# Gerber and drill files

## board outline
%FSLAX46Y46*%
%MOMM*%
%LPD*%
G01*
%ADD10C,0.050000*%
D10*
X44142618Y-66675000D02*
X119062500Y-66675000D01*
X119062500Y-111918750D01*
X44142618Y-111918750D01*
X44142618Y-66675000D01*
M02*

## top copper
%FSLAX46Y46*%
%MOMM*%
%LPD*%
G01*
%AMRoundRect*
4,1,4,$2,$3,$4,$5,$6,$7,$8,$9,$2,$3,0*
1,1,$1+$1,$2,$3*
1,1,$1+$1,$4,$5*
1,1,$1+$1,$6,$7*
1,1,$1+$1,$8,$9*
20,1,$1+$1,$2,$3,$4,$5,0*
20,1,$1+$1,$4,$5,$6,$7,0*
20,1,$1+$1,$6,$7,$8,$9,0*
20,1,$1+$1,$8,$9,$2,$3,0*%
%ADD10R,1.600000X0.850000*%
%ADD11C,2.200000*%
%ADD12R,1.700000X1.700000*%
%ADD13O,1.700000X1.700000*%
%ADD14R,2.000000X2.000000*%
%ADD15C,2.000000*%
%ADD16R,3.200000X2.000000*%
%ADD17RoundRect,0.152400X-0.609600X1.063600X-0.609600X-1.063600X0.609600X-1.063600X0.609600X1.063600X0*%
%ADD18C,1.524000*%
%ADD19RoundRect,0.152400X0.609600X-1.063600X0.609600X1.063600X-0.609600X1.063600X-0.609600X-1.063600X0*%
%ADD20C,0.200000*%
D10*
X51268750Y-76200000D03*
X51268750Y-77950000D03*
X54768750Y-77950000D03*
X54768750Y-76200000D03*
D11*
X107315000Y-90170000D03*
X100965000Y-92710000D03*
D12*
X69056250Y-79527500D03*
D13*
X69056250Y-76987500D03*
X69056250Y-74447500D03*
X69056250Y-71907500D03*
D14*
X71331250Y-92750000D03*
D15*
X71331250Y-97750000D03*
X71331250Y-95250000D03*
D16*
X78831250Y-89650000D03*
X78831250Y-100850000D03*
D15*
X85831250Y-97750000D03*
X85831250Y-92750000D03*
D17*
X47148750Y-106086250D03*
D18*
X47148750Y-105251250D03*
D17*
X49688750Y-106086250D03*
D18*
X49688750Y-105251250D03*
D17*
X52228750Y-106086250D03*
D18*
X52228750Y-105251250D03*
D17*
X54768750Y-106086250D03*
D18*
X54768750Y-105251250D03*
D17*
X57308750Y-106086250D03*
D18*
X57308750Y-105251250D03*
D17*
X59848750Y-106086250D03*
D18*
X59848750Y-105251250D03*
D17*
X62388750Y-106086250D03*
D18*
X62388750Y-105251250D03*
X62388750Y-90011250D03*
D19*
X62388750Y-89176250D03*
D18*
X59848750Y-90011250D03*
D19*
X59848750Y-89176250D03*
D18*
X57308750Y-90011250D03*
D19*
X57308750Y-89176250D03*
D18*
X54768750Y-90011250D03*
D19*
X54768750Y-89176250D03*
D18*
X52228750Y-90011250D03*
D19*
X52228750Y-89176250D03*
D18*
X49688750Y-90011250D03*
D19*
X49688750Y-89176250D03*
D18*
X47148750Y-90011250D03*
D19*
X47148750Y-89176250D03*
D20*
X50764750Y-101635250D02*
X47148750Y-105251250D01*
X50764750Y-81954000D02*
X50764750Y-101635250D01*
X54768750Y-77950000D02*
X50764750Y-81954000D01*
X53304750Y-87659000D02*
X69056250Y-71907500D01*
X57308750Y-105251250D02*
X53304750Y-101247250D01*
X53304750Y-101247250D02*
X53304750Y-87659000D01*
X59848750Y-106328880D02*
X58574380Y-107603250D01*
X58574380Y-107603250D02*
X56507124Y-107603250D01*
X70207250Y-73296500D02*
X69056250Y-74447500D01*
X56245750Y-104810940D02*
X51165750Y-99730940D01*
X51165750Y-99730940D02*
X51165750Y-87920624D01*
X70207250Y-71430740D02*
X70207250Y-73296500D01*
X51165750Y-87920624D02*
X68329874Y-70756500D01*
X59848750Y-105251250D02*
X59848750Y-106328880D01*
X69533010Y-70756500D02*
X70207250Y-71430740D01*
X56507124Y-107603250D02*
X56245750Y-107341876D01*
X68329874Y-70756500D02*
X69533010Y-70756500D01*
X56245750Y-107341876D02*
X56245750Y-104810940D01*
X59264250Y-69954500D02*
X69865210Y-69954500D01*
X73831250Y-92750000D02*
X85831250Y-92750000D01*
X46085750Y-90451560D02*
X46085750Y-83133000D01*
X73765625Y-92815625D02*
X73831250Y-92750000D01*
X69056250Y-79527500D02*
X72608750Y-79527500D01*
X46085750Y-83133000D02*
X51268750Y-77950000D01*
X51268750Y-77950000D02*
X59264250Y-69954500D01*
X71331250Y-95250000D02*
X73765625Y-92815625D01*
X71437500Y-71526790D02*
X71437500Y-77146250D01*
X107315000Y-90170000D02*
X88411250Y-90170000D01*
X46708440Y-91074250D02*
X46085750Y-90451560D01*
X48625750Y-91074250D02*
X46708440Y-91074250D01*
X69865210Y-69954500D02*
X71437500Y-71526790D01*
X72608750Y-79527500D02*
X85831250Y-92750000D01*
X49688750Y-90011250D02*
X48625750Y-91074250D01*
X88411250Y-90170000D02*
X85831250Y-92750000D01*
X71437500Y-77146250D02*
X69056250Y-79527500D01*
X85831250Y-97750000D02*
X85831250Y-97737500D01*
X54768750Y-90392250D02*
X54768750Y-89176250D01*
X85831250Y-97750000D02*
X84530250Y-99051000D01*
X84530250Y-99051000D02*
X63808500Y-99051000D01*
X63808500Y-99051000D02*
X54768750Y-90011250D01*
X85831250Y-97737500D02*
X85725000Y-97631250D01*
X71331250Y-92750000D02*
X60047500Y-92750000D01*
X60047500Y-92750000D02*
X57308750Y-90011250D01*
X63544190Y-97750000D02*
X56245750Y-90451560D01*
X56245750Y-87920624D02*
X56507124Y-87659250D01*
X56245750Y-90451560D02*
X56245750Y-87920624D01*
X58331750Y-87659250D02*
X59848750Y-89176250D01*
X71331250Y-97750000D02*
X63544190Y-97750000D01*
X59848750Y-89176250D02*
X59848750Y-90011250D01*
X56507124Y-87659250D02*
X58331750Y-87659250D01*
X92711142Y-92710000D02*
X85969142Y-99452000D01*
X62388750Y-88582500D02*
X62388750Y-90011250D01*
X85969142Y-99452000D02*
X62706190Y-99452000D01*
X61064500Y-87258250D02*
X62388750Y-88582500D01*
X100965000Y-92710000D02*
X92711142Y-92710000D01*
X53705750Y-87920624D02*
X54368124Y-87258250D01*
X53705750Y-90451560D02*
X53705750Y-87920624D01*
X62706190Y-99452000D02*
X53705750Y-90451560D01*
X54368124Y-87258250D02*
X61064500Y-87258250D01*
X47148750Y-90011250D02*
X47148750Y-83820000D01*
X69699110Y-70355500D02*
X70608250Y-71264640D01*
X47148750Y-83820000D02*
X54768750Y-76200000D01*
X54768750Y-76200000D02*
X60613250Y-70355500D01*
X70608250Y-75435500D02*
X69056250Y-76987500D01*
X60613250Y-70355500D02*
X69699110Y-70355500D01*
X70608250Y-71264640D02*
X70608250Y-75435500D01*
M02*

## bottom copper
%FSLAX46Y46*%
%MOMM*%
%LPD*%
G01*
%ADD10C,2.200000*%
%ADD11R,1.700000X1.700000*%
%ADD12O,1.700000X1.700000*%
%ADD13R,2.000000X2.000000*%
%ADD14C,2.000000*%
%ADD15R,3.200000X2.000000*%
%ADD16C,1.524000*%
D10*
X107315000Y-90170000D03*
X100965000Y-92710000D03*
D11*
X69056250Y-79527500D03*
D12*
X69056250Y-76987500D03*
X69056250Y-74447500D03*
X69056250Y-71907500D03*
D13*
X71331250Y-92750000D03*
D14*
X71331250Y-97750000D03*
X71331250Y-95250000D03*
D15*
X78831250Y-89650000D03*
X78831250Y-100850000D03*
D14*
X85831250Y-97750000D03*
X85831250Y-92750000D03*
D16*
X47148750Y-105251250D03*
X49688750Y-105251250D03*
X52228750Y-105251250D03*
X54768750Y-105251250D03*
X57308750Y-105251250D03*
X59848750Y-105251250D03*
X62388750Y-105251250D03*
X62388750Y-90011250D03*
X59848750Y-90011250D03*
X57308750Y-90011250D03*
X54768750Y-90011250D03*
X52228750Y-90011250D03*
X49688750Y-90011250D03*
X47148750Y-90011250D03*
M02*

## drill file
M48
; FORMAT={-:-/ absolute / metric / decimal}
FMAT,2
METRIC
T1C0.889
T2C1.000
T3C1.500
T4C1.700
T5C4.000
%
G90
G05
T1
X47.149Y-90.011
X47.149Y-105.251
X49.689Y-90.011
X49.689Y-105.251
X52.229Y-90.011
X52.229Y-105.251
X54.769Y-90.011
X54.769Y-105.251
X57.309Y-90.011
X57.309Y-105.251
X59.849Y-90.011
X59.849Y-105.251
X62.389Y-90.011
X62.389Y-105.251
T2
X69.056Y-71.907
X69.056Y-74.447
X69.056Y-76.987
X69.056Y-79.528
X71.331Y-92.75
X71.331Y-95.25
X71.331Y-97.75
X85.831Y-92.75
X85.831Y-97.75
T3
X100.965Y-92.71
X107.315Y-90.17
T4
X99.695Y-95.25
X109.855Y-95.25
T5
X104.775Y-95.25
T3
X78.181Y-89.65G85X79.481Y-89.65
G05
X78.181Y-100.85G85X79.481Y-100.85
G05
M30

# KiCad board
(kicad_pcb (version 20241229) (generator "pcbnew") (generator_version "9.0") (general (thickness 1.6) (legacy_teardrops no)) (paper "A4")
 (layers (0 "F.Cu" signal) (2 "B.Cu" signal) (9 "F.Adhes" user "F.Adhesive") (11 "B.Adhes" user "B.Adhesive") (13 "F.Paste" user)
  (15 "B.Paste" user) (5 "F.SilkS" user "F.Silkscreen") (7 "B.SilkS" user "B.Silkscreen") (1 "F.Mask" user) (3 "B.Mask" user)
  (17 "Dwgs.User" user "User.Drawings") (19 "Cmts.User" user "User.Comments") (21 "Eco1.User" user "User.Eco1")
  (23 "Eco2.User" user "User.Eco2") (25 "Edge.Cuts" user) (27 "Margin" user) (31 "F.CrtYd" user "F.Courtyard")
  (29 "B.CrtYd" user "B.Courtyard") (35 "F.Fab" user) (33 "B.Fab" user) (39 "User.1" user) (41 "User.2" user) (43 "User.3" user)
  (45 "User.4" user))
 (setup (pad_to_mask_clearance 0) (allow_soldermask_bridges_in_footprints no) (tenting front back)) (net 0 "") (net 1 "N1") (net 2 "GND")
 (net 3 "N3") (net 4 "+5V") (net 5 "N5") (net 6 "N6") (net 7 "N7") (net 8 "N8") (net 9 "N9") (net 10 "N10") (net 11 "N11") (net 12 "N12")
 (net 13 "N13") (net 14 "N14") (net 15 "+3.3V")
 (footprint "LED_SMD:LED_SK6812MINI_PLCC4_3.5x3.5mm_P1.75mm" (layer "F.Cu") (at 53.01875 77.075)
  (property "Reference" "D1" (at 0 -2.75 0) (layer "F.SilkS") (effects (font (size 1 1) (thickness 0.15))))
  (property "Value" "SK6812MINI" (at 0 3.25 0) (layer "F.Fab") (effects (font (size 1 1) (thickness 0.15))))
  (pad "1" smd rect (at -1.75 -0.875) (size 1.6 0.85) (layers "F.Cu" "F.Mask" "F.Paste") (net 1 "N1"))
  (pad "2" smd rect (at -1.75 0.875) (size 1.6 0.85) (layers "F.Cu" "F.Mask" "F.Paste") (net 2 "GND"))
  (pad "3" smd rect (at 1.75 0.875) (size 1.6 0.85) (layers "F.Cu" "F.Mask" "F.Paste") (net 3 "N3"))
  (pad "4" smd rect (at 1.75 -0.875) (size 1.6 0.85) (layers "F.Cu" "F.Mask" "F.Paste") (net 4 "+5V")))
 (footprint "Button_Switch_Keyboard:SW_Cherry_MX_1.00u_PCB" (layer "F.Cu") (at 107.315 90.17)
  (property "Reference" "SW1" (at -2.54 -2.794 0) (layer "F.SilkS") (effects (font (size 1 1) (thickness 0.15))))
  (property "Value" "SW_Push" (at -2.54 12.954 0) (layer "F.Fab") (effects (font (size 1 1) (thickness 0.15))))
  (pad "" np_thru_hole circle (at -7.62 5.08) (size 1.7 1.7) (drill 1.7) (layers "*.Cu" "*.Mask"))
  (pad "" np_thru_hole circle (at -2.54 5.08) (size 4 4) (drill 4) (layers "*.Cu" "*.Mask"))
  (pad "" np_thru_hole circle (at 2.54 5.08) (size 1.7 1.7) (drill 1.7) (layers "*.Cu" "*.Mask"))
  (pad "1" thru_hole circle (at 0 0) (size 2.2 2.2) (drill 1.5) (layers "*.Cu" "*.Mask") (remove_unused_layers no) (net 2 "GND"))
  (pad "2" thru_hole circle (at -6.35 2.54) (size 2.2 2.2) (drill 1.5) (layers "*.Cu" "*.Mask") (remove_unused_layers no) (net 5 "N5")))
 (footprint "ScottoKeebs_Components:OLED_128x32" (layer "F.Cu") (at 67.45625 69.7275)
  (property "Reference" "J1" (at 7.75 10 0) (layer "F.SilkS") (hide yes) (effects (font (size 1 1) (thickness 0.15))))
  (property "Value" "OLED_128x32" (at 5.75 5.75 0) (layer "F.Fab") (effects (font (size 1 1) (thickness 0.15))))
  (pad "1" thru_hole rect (at 1.6 9.8 180) (size 1.7 1.7) (drill 1) (layers "*.Cu" "*.Mask") (remove_unused_layers no) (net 2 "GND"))
  (pad "2" thru_hole oval (at 1.6 7.26 180) (size 1.7 1.7) (drill 1) (layers "*.Cu" "*.Mask") (remove_unused_layers no) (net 4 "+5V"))
  (pad "3" thru_hole oval (at 1.6 4.72 180) (size 1.7 1.7) (drill 1) (layers "*.Cu" "*.Mask") (remove_unused_layers no) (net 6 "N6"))
  (pad "4" thru_hole oval (at 1.6 2.18 180) (size 1.7 1.7) (drill 1) (layers "*.Cu" "*.Mask") (remove_unused_layers no) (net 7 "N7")))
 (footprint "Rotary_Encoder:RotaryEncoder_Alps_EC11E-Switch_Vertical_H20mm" (layer "F.Cu") (at 71.33125 92.75)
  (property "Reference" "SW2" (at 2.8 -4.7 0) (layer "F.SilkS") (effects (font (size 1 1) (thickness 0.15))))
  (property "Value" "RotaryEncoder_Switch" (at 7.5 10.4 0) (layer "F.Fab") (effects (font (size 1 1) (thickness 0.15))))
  (pad "A" thru_hole rect (at 0 0) (size 2 2) (drill 1) (layers "*.Cu" "*.Mask") (remove_unused_layers no) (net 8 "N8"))
  (pad "B" thru_hole circle (at 0 5) (size 2 2) (drill 1) (layers "*.Cu" "*.Mask") (remove_unused_layers no) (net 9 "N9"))
  (pad "C" thru_hole circle (at 0 2.5) (size 2 2) (drill 1) (layers "*.Cu" "*.Mask") (remove_unused_layers no) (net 2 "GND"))
  (pad "MP" thru_hole rect (at 7.5 -3.1) (size 3.2 2) (drill oval 2.8 1.5) (layers "*.Cu" "*.Mask") (remove_unused_layers no))
  (pad "MP" thru_hole rect (at 7.5 8.1) (size 3.2 2) (drill oval 2.8 1.5) (layers "*.Cu" "*.Mask") (remove_unused_layers no))
  (pad "S1" thru_hole circle (at 14.5 5) (size 2 2) (drill 1) (layers "*.Cu" "*.Mask") (remove_unused_layers no) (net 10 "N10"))
  (pad "S2" thru_hole circle (at 14.5 0) (size 2 2) (drill 1) (layers "*.Cu" "*.Mask") (remove_unused_layers no) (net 2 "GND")))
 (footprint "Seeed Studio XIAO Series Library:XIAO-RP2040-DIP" (layer "F.Cu") (at 54.76875 97.63125 90)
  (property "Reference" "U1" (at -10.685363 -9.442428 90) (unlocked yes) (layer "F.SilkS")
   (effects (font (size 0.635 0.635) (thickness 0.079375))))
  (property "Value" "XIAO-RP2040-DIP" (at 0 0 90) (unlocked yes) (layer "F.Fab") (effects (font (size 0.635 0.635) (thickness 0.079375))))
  (pad "1" smd roundrect (at -8.455 -7.62 270) (size 2.432 1.524) (layers "F.Cu" "F.Mask") (roundrect_rratio 0.1) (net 3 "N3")
   (thermal_bridge_angle 45))
  (pad "1" thru_hole circle (at -7.62 -7.62 270) (size 1.524 1.524) (drill 0.889) (layers "*.Cu" "*.Mask") (remove_unused_layers no)
   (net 3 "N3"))
  (pad "2" smd roundrect (at -8.455 -5.08 270) (size 2.432 1.524) (layers "F.Cu" "F.Mask") (roundrect_rratio 0.1) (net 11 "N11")
   (thermal_bridge_angle 45))
  (pad "2" thru_hole circle (at -7.62 -5.08 270) (size 1.524 1.524) (drill 0.889) (layers "*.Cu" "*.Mask") (remove_unused_layers no)
   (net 11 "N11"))
  (pad "3" smd roundrect (at -8.455 -2.54 270) (size 2.432 1.524) (layers "F.Cu" "F.Mask") (roundrect_rratio 0.1) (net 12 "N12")
   (thermal_bridge_angle 45))
  (pad "3" thru_hole circle (at -7.62 -2.54 270) (size 1.524 1.524) (drill 0.889) (layers "*.Cu" "*.Mask") (remove_unused_layers no)
   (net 12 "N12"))
  (pad "4" smd roundrect (at -8.455 0 270) (size 2.432 1.524) (layers "F.Cu" "F.Mask") (roundrect_rratio 0.1) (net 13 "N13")
   (thermal_bridge_angle 45))
  (pad "4" thru_hole circle (at -7.62 0 270) (size 1.524 1.524) (drill 0.889) (layers "*.Cu" "*.Mask") (remove_unused_layers no)
   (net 13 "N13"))
  (pad "5" smd roundrect (at -8.455 2.54 270) (size 2.432 1.524) (layers "F.Cu" "F.Mask") (roundrect_rratio 0.1) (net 7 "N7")
   (thermal_bridge_angle 45))
  (pad "5" thru_hole circle (at -7.62 2.54 270) (size 1.524 1.524) (drill 0.889) (layers "*.Cu" "*.Mask") (remove_unused_layers no)
   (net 7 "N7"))
  (pad "6" smd roundrect (at -8.455 5.08 270) (size 2.432 1.524) (layers "F.Cu" "F.Mask") (roundrect_rratio 0.1) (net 6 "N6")
   (thermal_bridge_angle 45))
  (pad "6" thru_hole circle (at -7.62 5.08 270) (size 1.524 1.524) (drill 0.889) (layers "*.Cu" "*.Mask") (remove_unused_layers no)
   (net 6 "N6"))
  (pad "7" smd roundrect (at -8.455 7.62 270) (size 2.432 1.524) (layers "F.Cu" "F.Mask") (roundrect_rratio 0.1) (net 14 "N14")
   (thermal_bridge_angle 45))
  (pad "7" thru_hole circle (at -7.62 7.62 270) (size 1.524 1.524) (drill 0.889) (layers "*.Cu" "*.Mask") (remove_unused_layers no)
   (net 14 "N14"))
  (pad "8" thru_hole circle (at 7.62 7.62 90) (size 1.524 1.524) (drill 0.889) (layers "*.Cu" "*.Mask") (remove_unused_layers no)
   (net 5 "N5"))
  (pad "8" smd roundrect (at 8.455 7.62 90) (size 2.432 1.524) (layers "F.Cu" "F.Mask") (roundrect_rratio 0.1) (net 5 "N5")
   (thermal_bridge_angle 45))
  (pad "9" thru_hole circle (at 7.62 5.08 90) (size 1.524 1.524) (drill 0.889) (layers "*.Cu" "*.Mask") (remove_unused_layers no)
   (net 9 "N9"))
  (pad "9" smd roundrect (at 8.455 5.08 90) (size 2.432 1.524) (layers "F.Cu" "F.Mask") (roundrect_rratio 0.1) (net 9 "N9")
   (thermal_bridge_angle 45))
  (pad "10" thru_hole circle (at 7.62 2.54 90) (size 1.524 1.524) (drill 0.889) (layers "*.Cu" "*.Mask") (remove_unused_layers no)
   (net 8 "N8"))
  (pad "10" smd roundrect (at 8.455 2.54 90) (size 2.432 1.524) (layers "F.Cu" "F.Mask") (roundrect_rratio 0.1) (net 8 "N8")
   (thermal_bridge_angle 45))
  (pad "11" thru_hole circle (at 7.62 0 90) (size 1.524 1.524) (drill 0.889) (layers "*.Cu" "*.Mask") (remove_unused_layers no)
   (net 10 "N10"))
  (pad "11" smd roundrect (at 8.455 0 90) (size 2.432 1.524) (layers "F.Cu" "F.Mask") (roundrect_rratio 0.1) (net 10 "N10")
   (thermal_bridge_angle 45))
  (pad "12" thru_hole circle (at 7.62 -2.54 90) (size 1.524 1.524) (drill 0.889) (layers "*.Cu" "*.Mask") (remove_unused_layers no)
   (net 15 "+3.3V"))
  (pad "12" smd roundrect (at 8.455 -2.54 90) (size 2.432 1.524) (layers "F.Cu" "F.Mask") (roundrect_rratio 0.1) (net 15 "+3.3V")
   (thermal_bridge_angle 45))
  (pad "13" thru_hole circle (at 7.62 -5.08 90) (size 1.524 1.524) (drill 0.889) (layers "*.Cu" "*.Mask") (remove_unused_layers no)
   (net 2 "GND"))
  (pad "13" smd roundrect (at 8.455 -5.08 90) (size 2.432 1.524) (layers "F.Cu" "F.Mask") (roundrect_rratio 0.1) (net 2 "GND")
   (thermal_bridge_angle 45))
  (pad "14" thru_hole circle (at 7.62 -7.62 90) (size 1.524 1.524) (drill 0.889) (layers "*.Cu" "*.Mask") (remove_unused_layers no)
   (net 4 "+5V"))
  (pad "14" smd roundrect (at 8.455 -7.62 90) (size 2.432 1.524) (layers "F.Cu" "F.Mask") (roundrect_rratio 0.1) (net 4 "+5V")
   (thermal_bridge_angle 45)))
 (gr_rect (start 44.142618 66.675) (end 119.0625 111.91875) (stroke (width 0.05) (type default)) (fill no) (layer "Edge.Cuts"))
 (segment (start 50.76475 101.63525) (end 47.14875 105.25125) (width 0.2) (layer "F.Cu") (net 3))
 (segment (start 50.76475 81.954) (end 50.76475 101.63525) (width 0.2) (layer "F.Cu") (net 3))
 (segment (start 54.76875 77.95) (end 50.76475 81.954) (width 0.2) (layer "F.Cu") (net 3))
 (segment (start 53.30475 87.659) (end 69.05625 71.9075) (width 0.2) (layer "F.Cu") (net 7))
 (segment (start 57.30875 105.25125) (end 53.30475 101.24725) (width 0.2) (layer "F.Cu") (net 7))
 (segment (start 53.30475 101.24725) (end 53.30475 87.659) (width 0.2) (layer "F.Cu") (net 7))
 (segment (start 59.84875 106.32888) (end 58.57438 107.60325) (width 0.2) (layer "F.Cu") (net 6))
 (segment (start 58.57438 107.60325) (end 56.507124 107.60325) (width 0.2) (layer "F.Cu") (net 6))
 (segment (start 70.20725 73.2965) (end 69.05625 74.4475) (width 0.2) (layer "F.Cu") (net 6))
 (segment (start 56.24575 104.81094) (end 51.16575 99.73094) (width 0.2) (layer "F.Cu") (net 6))
 (segment (start 51.16575 99.73094) (end 51.16575 87.920624) (width 0.2) (layer "F.Cu") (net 6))
 (segment (start 70.20725 71.43074) (end 70.20725 73.2965) (width 0.2) (layer "F.Cu") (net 6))
 (segment (start 51.16575 87.920624) (end 68.329874 70.7565) (width 0.2) (layer "F.Cu") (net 6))
 (segment (start 59.84875 105.25125) (end 59.84875 106.32888) (width 0.2) (layer "F.Cu") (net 6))
 (segment (start 69.53301 70.7565) (end 70.20725 71.43074) (width 0.2) (layer "F.Cu") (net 6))
 (segment (start 56.507124 107.60325) (end 56.24575 107.341876) (width 0.2) (layer "F.Cu") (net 6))
 (segment (start 68.329874 70.7565) (end 69.53301 70.7565) (width 0.2) (layer "F.Cu") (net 6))
 (segment (start 56.24575 107.341876) (end 56.24575 104.81094) (width 0.2) (layer "F.Cu") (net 6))
 (segment (start 59.26425 69.9545) (end 69.86521 69.9545) (width 0.2) (layer "F.Cu") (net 2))
 (segment (start 73.83125 92.75) (end 85.83125 92.75) (width 0.2) (layer "F.Cu") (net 2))
 (segment (start 46.08575 90.45156) (end 46.08575 83.133) (width 0.2) (layer "F.Cu") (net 2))
 (segment (start 73.765625 92.815625) (end 73.83125 92.75) (width 0.2) (layer "F.Cu") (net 2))
 (segment (start 69.05625 79.5275) (end 72.60875 79.5275) (width 0.2) (layer "F.Cu") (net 2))
 (segment (start 46.08575 83.133) (end 51.26875 77.95) (width 0.2) (layer "F.Cu") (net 2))
 (segment (start 51.26875 77.95) (end 59.26425 69.9545) (width 0.2) (layer "F.Cu") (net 2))
 (segment (start 71.33125 95.25) (end 73.765625 92.815625) (width 0.2) (layer "F.Cu") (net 2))
 (segment (start 71.4375 71.52679) (end 71.4375 77.14625) (width 0.2) (layer "F.Cu") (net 2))
 (segment (start 107.315 90.17) (end 88.41125 90.17) (width 0.2) (layer "F.Cu") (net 2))
 (segment (start 46.70844 91.07425) (end 46.08575 90.45156) (width 0.2) (layer "F.Cu") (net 2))
 (segment (start 48.62575 91.07425) (end 46.70844 91.07425) (width 0.2) (layer "F.Cu") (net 2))
 (segment (start 69.86521 69.9545) (end 71.4375 71.52679) (width 0.2) (layer "F.Cu") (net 2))
 (segment (start 72.60875 79.5275) (end 85.83125 92.75) (width 0.2) (layer "F.Cu") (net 2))
 (segment (start 49.68875 90.01125) (end 48.62575 91.07425) (width 0.2) (layer "F.Cu") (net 2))
 (segment (start 88.41125 90.17) (end 85.83125 92.75) (width 0.2) (layer "F.Cu") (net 2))
 (segment (start 71.4375 77.14625) (end 69.05625 79.5275) (width 0.2) (layer "F.Cu") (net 2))
 (segment (start 85.83125 97.75) (end 85.83125 97.7375) (width 0.2) (layer "F.Cu") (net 10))
 (segment (start 54.76875 90.39225) (end 54.76875 89.17625) (width 0.2) (layer "F.Cu") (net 10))
 (segment (start 85.83125 97.75) (end 84.53025 99.051) (width 0.2) (layer "F.Cu") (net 10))
 (segment (start 84.53025 99.051) (end 63.8085 99.051) (width 0.2) (layer "F.Cu") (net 10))
 (segment (start 63.8085 99.051) (end 54.76875 90.01125) (width 0.2) (layer "F.Cu") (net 10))
 (segment (start 85.83125 97.7375) (end 85.725 97.63125) (width 0.2) (layer "F.Cu") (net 10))
 (segment (start 71.33125 92.75) (end 60.0475 92.75) (width 0.2) (layer "F.Cu") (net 8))
 (segment (start 60.0475 92.75) (end 57.30875 90.01125) (width 0.2) (layer "F.Cu") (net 8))
 (segment (start 63.54419 97.75) (end 56.24575 90.45156) (width 0.2) (layer "F.Cu") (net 9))
 (segment (start 56.24575 87.920624) (end 56.507124 87.65925) (width 0.2) (layer "F.Cu") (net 9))
 (segment (start 56.24575 90.45156) (end 56.24575 87.920624) (width 0.2) (layer "F.Cu") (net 9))
 (segment (start 58.33175 87.65925) (end 59.84875 89.17625) (width 0.2) (layer "F.Cu") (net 9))
 (segment (start 71.33125 97.75) (end 63.54419 97.75) (width 0.2) (layer "F.Cu") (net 9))
 (segment (start 59.84875 89.17625) (end 59.84875 90.01125) (width 0.2) (layer "F.Cu") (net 9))
 (segment (start 56.507124 87.65925) (end 58.33175 87.65925) (width 0.2) (layer "F.Cu") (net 9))
 (segment (start 92.711142 92.71) (end 85.969142 99.452) (width 0.2) (layer "F.Cu") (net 5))
 (segment (start 62.38875 88.5825) (end 62.38875 90.01125) (width 0.2) (layer "F.Cu") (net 5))
 (segment (start 85.969142 99.452) (end 62.70619 99.452) (width 0.2) (layer "F.Cu") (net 5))
 (segment (start 61.0645 87.25825) (end 62.38875 88.5825) (width 0.2) (layer "F.Cu") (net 5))
 (segment (start 100.965 92.71) (end 92.711142 92.71) (width 0.2) (layer "F.Cu") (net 5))
 (segment (start 53.70575 87.920624) (end 54.368124 87.25825) (width 0.2) (layer "F.Cu") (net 5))
 (segment (start 53.70575 90.45156) (end 53.70575 87.920624) (width 0.2) (layer "F.Cu") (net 5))
 (segment (start 62.70619 99.452) (end 53.70575 90.45156) (width 0.2) (layer "F.Cu") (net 5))
 (segment (start 54.368124 87.25825) (end 61.0645 87.25825) (width 0.2) (layer "F.Cu") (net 5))
 (segment (start 47.14875 90.01125) (end 47.14875 83.82) (width 0.2) (layer "F.Cu") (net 4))
 (segment (start 69.69911 70.3555) (end 70.60825 71.26464) (width 0.2) (layer "F.Cu") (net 4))
 (segment (start 47.14875 83.82) (end 54.76875 76.2) (width 0.2) (layer "F.Cu") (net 4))
 (segment (start 54.76875 76.2) (end 60.61325 70.3555) (width 0.2) (layer "F.Cu") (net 4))
 (segment (start 70.60825 75.4355) (end 69.05625 76.9875) (width 0.2) (layer "F.Cu") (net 4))
 (segment (start 60.61325 70.3555) (end 69.69911 70.3555) (width 0.2) (layer "F.Cu") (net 4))
 (segment (start 70.60825 71.26464) (end 70.60825 75.4355) (width 0.2) (layer "F.Cu") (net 4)))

